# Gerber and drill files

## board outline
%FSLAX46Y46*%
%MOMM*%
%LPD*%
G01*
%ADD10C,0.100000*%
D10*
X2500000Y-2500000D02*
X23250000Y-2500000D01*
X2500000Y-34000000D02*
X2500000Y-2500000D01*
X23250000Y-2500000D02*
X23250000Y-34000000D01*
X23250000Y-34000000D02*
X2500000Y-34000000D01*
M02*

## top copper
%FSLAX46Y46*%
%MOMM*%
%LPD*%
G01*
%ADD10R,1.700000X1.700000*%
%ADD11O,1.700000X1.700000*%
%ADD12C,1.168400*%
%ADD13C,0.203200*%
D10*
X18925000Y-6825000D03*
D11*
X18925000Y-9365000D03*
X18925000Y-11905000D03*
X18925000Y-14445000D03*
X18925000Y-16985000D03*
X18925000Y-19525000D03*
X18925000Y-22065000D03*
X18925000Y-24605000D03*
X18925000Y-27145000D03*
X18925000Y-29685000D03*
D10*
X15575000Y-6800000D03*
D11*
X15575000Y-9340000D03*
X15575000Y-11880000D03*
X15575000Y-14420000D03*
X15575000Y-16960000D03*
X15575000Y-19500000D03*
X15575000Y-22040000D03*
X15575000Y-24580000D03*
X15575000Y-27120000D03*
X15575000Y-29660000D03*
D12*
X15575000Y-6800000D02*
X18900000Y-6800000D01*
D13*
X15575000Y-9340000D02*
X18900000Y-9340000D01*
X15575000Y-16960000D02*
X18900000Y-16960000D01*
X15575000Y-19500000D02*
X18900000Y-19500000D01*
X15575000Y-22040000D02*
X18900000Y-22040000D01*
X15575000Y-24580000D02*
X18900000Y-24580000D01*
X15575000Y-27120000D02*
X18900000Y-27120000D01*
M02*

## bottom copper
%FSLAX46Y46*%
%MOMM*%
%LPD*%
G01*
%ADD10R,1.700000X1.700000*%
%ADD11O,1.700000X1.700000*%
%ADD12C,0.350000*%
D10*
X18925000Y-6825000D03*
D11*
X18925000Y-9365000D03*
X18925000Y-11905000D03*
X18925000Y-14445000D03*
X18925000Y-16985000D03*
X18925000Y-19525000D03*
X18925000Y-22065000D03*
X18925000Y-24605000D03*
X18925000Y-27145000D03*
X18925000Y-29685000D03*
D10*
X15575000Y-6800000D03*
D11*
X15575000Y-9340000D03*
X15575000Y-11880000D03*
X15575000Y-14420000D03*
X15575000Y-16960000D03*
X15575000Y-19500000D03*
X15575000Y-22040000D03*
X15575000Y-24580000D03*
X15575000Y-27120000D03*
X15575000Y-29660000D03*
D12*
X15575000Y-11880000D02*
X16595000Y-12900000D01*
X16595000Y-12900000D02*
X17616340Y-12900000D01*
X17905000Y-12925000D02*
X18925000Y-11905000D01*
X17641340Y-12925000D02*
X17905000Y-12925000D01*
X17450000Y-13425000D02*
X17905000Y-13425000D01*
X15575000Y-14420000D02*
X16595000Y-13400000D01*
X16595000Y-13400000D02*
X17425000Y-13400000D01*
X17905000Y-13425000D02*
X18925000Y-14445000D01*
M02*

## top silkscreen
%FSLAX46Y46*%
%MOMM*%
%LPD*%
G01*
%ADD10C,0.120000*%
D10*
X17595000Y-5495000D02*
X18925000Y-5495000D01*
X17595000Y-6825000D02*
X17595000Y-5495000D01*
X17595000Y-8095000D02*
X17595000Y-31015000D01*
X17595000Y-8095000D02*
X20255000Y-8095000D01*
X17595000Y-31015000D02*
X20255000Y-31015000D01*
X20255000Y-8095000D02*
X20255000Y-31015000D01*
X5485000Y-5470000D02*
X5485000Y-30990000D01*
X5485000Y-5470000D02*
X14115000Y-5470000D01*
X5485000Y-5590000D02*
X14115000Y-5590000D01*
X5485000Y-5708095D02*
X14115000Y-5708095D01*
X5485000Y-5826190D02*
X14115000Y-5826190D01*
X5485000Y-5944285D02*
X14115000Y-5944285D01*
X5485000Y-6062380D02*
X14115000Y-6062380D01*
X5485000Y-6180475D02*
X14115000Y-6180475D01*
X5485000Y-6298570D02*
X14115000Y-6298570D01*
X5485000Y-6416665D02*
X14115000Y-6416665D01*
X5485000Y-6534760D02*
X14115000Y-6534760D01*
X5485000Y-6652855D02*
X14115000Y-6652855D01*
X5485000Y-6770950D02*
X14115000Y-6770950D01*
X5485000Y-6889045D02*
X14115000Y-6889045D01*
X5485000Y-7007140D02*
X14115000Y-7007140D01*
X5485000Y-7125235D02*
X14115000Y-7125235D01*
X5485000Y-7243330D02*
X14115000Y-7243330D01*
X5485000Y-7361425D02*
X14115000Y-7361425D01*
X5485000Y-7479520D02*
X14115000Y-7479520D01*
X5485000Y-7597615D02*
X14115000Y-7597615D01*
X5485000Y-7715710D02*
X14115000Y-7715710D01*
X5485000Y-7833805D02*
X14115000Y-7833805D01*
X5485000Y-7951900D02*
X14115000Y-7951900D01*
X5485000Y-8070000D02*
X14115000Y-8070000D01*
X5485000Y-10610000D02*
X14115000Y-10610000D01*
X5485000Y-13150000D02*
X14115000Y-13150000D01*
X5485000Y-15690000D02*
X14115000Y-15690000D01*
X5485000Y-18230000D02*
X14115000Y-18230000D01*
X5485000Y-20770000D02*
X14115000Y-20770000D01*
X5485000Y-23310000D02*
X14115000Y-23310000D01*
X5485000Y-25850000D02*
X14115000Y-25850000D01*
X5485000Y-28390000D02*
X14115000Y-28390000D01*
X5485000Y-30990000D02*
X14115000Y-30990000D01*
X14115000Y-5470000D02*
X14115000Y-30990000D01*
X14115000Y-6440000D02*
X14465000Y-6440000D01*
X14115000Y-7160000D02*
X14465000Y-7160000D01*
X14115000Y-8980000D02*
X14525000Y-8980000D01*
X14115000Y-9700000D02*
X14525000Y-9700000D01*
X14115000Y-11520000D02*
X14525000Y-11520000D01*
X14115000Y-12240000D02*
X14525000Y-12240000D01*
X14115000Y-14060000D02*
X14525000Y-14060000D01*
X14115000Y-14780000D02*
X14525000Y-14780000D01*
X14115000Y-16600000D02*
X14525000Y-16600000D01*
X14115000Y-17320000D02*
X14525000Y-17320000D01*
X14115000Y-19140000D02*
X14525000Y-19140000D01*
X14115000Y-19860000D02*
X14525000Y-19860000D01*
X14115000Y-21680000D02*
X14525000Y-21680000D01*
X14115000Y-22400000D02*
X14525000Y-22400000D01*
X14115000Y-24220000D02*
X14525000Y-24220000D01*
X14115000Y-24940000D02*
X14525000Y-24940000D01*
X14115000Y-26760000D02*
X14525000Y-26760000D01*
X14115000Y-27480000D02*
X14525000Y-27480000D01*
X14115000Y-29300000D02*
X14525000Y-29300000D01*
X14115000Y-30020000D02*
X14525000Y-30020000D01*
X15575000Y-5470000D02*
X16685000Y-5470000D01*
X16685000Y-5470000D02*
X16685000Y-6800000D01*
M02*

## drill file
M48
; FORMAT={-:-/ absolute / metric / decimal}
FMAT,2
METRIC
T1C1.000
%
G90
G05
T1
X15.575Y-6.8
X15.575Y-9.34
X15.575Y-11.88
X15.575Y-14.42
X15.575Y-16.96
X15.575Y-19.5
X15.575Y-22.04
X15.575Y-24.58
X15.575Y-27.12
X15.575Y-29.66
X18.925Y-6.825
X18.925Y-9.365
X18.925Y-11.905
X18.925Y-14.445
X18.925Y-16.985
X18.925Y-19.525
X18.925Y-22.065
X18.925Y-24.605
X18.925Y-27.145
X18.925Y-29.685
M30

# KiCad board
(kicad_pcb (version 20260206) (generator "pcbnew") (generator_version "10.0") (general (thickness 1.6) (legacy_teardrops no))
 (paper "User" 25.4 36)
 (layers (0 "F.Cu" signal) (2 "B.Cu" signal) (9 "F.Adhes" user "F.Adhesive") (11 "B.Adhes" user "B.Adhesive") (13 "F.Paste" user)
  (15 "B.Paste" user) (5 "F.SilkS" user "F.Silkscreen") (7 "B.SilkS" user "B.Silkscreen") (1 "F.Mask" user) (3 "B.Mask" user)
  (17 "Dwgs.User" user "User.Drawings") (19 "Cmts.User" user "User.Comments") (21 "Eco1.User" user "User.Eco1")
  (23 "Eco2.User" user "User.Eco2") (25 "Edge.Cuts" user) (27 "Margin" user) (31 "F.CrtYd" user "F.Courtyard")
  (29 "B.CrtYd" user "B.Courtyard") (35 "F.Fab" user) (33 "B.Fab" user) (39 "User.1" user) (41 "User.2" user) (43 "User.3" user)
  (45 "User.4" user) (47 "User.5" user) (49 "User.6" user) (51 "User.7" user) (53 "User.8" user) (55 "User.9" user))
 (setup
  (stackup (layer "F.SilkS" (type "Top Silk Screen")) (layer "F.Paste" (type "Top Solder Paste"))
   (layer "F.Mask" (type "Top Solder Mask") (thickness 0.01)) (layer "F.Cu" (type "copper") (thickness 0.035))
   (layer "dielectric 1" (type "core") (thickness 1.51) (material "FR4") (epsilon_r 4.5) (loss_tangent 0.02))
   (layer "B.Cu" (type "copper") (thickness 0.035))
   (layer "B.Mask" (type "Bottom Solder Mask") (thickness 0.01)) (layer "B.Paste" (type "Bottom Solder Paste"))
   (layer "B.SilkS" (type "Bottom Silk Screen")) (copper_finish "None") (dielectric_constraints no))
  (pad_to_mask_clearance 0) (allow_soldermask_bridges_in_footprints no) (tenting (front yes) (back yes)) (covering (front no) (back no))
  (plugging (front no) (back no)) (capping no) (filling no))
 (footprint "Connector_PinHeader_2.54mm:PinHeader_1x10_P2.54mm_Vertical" (layer "F.Cu") (at 18.925 6.825)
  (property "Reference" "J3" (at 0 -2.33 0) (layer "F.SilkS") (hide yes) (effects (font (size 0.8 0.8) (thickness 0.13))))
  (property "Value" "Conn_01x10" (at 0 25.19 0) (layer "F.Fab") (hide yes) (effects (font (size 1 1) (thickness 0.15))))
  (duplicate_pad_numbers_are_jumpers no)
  (fp_line (start -1.33 -1.33) (end 0 -1.33) (stroke (width 0.12) (type solid)) (layer "F.SilkS"))
  (fp_line (start -1.33 0) (end -1.33 -1.33) (stroke (width 0.12) (type solid)) (layer "F.SilkS"))
  (fp_line (start -1.33 1.27) (end -1.33 24.19) (stroke (width 0.12) (type solid)) (layer "F.SilkS"))
  (fp_line (start -1.33 1.27) (end 1.33 1.27) (stroke (width 0.12) (type solid)) (layer "F.SilkS"))
  (fp_line (start -1.33 24.19) (end 1.33 24.19) (stroke (width 0.12) (type solid)) (layer "F.SilkS"))
  (fp_line (start 1.33 1.27) (end 1.33 24.19) (stroke (width 0.12) (type solid)) (layer "F.SilkS"))
  (pad "1" thru_hole rect (at 0 0) (size 1.7 1.7) (drill 1) (layers "*.Cu" "*.Mask") (remove_unused_layers no) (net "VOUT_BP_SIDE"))
  (pad "2" thru_hole oval (at 0 2.54) (size 1.7 1.7) (drill 1) (layers "*.Cu" "*.Mask") (remove_unused_layers no) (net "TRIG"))
  (pad "3" thru_hole oval (at 0 5.08) (size 1.7 1.7) (drill 1) (layers "*.Cu" "*.Mask") (remove_unused_layers no) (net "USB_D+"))
  (pad "4" thru_hole oval (at 0 7.62) (size 1.7 1.7) (drill 1) (layers "*.Cu" "*.Mask") (remove_unused_layers no) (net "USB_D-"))
  (pad "5" thru_hole oval (at 0 10.16) (size 1.7 1.7) (drill 1) (layers "*.Cu" "*.Mask") (remove_unused_layers no) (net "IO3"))
  (pad "6" thru_hole oval (at 0 12.7) (size 1.7 1.7) (drill 1) (layers "*.Cu" "*.Mask") (remove_unused_layers no) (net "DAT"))
  (pad "7" thru_hole oval (at 0 15.24) (size 1.7 1.7) (drill 1) (layers "*.Cu" "*.Mask") (remove_unused_layers no) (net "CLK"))
  (pad "8" thru_hole oval (at 0 17.78) (size 1.7 1.7) (drill 1) (layers "*.Cu" "*.Mask") (remove_unused_layers no) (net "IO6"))
  (pad "9" thru_hole oval (at 0 20.32) (size 1.7 1.7) (drill 1) (layers "*.Cu" "*.Mask") (remove_unused_layers no) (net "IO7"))
  (pad "10" thru_hole oval (at 0 22.86) (size 1.7 1.7) (drill 1) (layers "*.Cu" "*.Mask") (remove_unused_layers no) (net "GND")))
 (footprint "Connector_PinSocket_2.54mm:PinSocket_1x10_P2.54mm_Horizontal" (layer "F.Cu") (at 15.575 6.8)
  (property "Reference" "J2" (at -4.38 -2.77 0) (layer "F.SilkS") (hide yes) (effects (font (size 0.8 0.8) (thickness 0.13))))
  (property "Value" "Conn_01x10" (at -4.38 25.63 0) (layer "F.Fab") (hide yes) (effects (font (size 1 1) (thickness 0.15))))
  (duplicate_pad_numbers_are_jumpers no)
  (fp_line (start -10.09 -1.33) (end -10.09 24.19) (stroke (width 0.12) (type solid)) (layer "F.SilkS"))
  (fp_line (start -10.09 -1.33) (end -1.46 -1.33) (stroke (width 0.12) (type solid)) (layer "F.SilkS"))
  (fp_line (start -10.09 -1.21) (end -1.46 -1.21) (stroke (width 0.12) (type solid)) (layer "F.SilkS"))
  (fp_line (start -10.09 -1.091905) (end -1.46 -1.091905) (stroke (width 0.12) (type solid)) (layer "F.SilkS"))
  (fp_line (start -10.09 -0.97381) (end -1.46 -0.97381) (stroke (width 0.12) (type solid)) (layer "F.SilkS"))
  (fp_line (start -10.09 -0.855715) (end -1.46 -0.855715) (stroke (width 0.12) (type solid)) (layer "F.SilkS"))
  (fp_line (start -10.09 -0.73762) (end -1.46 -0.73762) (stroke (width 0.12) (type solid)) (layer "F.SilkS"))
  (fp_line (start -10.09 -0.619525) (end -1.46 -0.619525) (stroke (width 0.12) (type solid)) (layer "F.SilkS"))
  (fp_line (start -10.09 -0.50143) (end -1.46 -0.50143) (stroke (width 0.12) (type solid)) (layer "F.SilkS"))
  (fp_line (start -10.09 -0.383335) (end -1.46 -0.383335) (stroke (width 0.12) (type solid)) (layer "F.SilkS"))
  (fp_line (start -10.09 -0.26524) (end -1.46 -0.26524) (stroke (width 0.12) (type solid)) (layer "F.SilkS"))
  (fp_line (start -10.09 -0.147145) (end -1.46 -0.147145) (stroke (width 0.12) (type solid)) (layer "F.SilkS"))
  (fp_line (start -10.09 -0.02905) (end -1.46 -0.02905) (stroke (width 0.12) (type solid)) (layer "F.SilkS"))
  (fp_line (start -10.09 0.089045) (end -1.46 0.089045) (stroke (width 0.12) (type solid)) (layer "F.SilkS"))
  (fp_line (start -10.09 0.20714) (end -1.46 0.20714) (stroke (width 0.12) (type solid)) (layer "F.SilkS"))
  (fp_line (start -10.09 0.325235) (end -1.46 0.325235) (stroke (width 0.12) (type solid)) (layer "F.SilkS"))
  (fp_line (start -10.09 0.44333) (end -1.46 0.44333) (stroke (width 0.12) (type solid)) (layer "F.SilkS"))
  (fp_line (start -10.09 0.561425) (end -1.46 0.561425) (stroke (width 0.12) (type solid)) (layer "F.SilkS"))
  (fp_line (start -10.09 0.67952) (end -1.46 0.67952) (stroke (width 0.12) (type solid)) (layer "F.SilkS"))
  (fp_line (start -10.09 0.797615) (end -1.46 0.797615) (stroke (width 0.12) (type solid)) (layer "F.SilkS"))
  (fp_line (start -10.09 0.91571) (end -1.46 0.91571) (stroke (width 0.12) (type solid)) (layer "F.SilkS"))
  (fp_line (start -10.09 1.033805) (end -1.46 1.033805) (stroke (width 0.12) (type solid)) (layer "F.SilkS"))
  (fp_line (start -10.09 1.1519) (end -1.46 1.1519) (stroke (width 0.12) (type solid)) (layer "F.SilkS"))
  (fp_line (start -10.09 1.27) (end -1.46 1.27) (stroke (width 0.12) (type solid)) (layer "F.SilkS"))
  (fp_line (start -10.09 3.81) (end -1.46 3.81) (stroke (width 0.12) (type solid)) (layer "F.SilkS"))
  (fp_line (start -10.09 6.35) (end -1.46 6.35) (stroke (width 0.12) (type solid)) (layer "F.SilkS"))
  (fp_line (start -10.09 8.89) (end -1.46 8.89) (stroke (width 0.12) (type solid)) (layer "F.SilkS"))
  (fp_line (start -10.09 11.43) (end -1.46 11.43) (stroke (width 0.12) (type solid)) (layer "F.SilkS"))
  (fp_line (start -10.09 13.97) (end -1.46 13.97) (stroke (width 0.12) (type solid)) (layer "F.SilkS"))
  (fp_line (start -10.09 16.51) (end -1.46 16.51) (stroke (width 0.12) (type solid)) (layer "F.SilkS"))
  (fp_line (start -10.09 19.05) (end -1.46 19.05) (stroke (width 0.12) (type solid)) (layer "F.SilkS"))
  (fp_line (start -10.09 21.59) (end -1.46 21.59) (stroke (width 0.12) (type solid)) (layer "F.SilkS"))
  (fp_line (start -10.09 24.19) (end -1.46 24.19) (stroke (width 0.12) (type solid)) (layer "F.SilkS"))
  (fp_line (start -1.46 -1.33) (end -1.46 24.19) (stroke (width 0.12) (type solid)) (layer "F.SilkS"))
  (fp_line (start -1.46 -0.36) (end -1.11 -0.36) (stroke (width 0.12) (type solid)) (layer "F.SilkS"))
  (fp_line (start -1.46 0.36) (end -1.11 0.36) (stroke (width 0.12) (type solid)) (layer "F.SilkS"))
  (fp_line (start -1.46 2.18) (end -1.05 2.18) (stroke (width 0.12) (type solid)) (layer "F.SilkS"))
  (fp_line (start -1.46 2.9) (end -1.05 2.9) (stroke (width 0.12) (type solid)) (layer "F.SilkS"))
  (fp_line (start -1.46 4.72) (end -1.05 4.72) (stroke (width 0.12) (type solid)) (layer "F.SilkS"))
  (fp_line (start -1.46 5.44) (end -1.05 5.44) (stroke (width 0.12) (type solid)) (layer "F.SilkS"))
  (fp_line (start -1.46 7.26) (end -1.05 7.26) (stroke (width 0.12) (type solid)) (layer "F.SilkS"))
  (fp_line (start -1.46 7.98) (end -1.05 7.98) (stroke (width 0.12) (type solid)) (layer "F.SilkS"))
  (fp_line (start -1.46 9.8) (end -1.05 9.8) (stroke (width 0.12) (type solid)) (layer "F.SilkS"))
  (fp_line (start -1.46 10.52) (end -1.05 10.52) (stroke (width 0.12) (type solid)) (layer "F.SilkS"))
  (fp_line (start -1.46 12.34) (end -1.05 12.34) (stroke (width 0.12) (type solid)) (layer "F.SilkS"))
  (fp_line (start -1.46 13.06) (end -1.05 13.06) (stroke (width 0.12) (type solid)) (layer "F.SilkS"))
  (fp_line (start -1.46 14.88) (end -1.05 14.88) (stroke (width 0.12) (type solid)) (layer "F.SilkS"))
  (fp_line (start -1.46 15.6) (end -1.05 15.6) (stroke (width 0.12) (type solid)) (layer "F.SilkS"))
  (fp_line (start -1.46 17.42) (end -1.05 17.42) (stroke (width 0.12) (type solid)) (layer "F.SilkS"))
  (fp_line (start -1.46 18.14) (end -1.05 18.14) (stroke (width 0.12) (type solid)) (layer "F.SilkS"))
  (fp_line (start -1.46 19.96) (end -1.05 19.96) (stroke (width 0.12) (type solid)) (layer "F.SilkS"))
  (fp_line (start -1.46 20.68) (end -1.05 20.68) (stroke (width 0.12) (type solid)) (layer "F.SilkS"))
  (fp_line (start -1.46 22.5) (end -1.05 22.5) (stroke (width 0.12) (type solid)) (layer "F.SilkS"))
  (fp_line (start -1.46 23.22) (end -1.05 23.22) (stroke (width 0.12) (type solid)) (layer "F.SilkS"))
  (fp_line (start 0 -1.33) (end 1.11 -1.33) (stroke (width 0.12) (type solid)) (layer "F.SilkS"))
  (fp_line (start 1.11 -1.33) (end 1.11 0) (stroke (width 0.12) (type solid)) (layer "F.SilkS"))
  (pad "1" thru_hole rect (at 0 0) (size 1.7 1.7) (drill 1) (layers "*.Cu" "*.Mask") (remove_unused_layers no) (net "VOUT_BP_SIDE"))
  (pad "2" thru_hole oval (at 0 2.54) (size 1.7 1.7) (drill 1) (layers "*.Cu" "*.Mask") (remove_unused_layers no) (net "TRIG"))
  (pad "3" thru_hole oval (at 0 5.08) (size 1.7 1.7) (drill 1) (layers "*.Cu" "*.Mask") (remove_unused_layers no) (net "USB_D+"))
  (pad "4" thru_hole oval (at 0 7.62) (size 1.7 1.7) (drill 1) (layers "*.Cu" "*.Mask") (remove_unused_layers no) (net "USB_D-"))
  (pad "5" thru_hole oval (at 0 10.16) (size 1.7 1.7) (drill 1) (layers "*.Cu" "*.Mask") (remove_unused_layers no) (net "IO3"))
  (pad "6" thru_hole oval (at 0 12.7) (size 1.7 1.7) (drill 1) (layers "*.Cu" "*.Mask") (remove_unused_layers no) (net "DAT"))
  (pad "7" thru_hole oval (at 0 15.24) (size 1.7 1.7) (drill 1) (layers "*.Cu" "*.Mask") (remove_unused_layers no) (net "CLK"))
  (pad "8" thru_hole oval (at 0 17.78) (size 1.7 1.7) (drill 1) (layers "*.Cu" "*.Mask") (remove_unused_layers no) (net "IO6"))
  (pad "9" thru_hole oval (at 0 20.32) (size 1.7 1.7) (drill 1) (layers "*.Cu" "*.Mask") (remove_unused_layers no) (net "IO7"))
  (pad "10" thru_hole oval (at 0 22.86) (size 1.7 1.7) (drill 1) (layers "*.Cu" "*.Mask") (remove_unused_layers no) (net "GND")))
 (gr_line (start 2.5 2.5) (end 23.25 2.5) (stroke (width 0.1) (type default)) (layer "Edge.Cuts"))
 (gr_line (start 2.5 34) (end 2.5 2.5) (stroke (width 0.1) (type default)) (layer "Edge.Cuts"))
 (gr_line (start 23.25 2.5) (end 23.25 34) (stroke (width 0.1) (type default)) (layer "Edge.Cuts"))
 (gr_line (start 23.25 34) (end 2.5 34) (stroke (width 0.1) (type default)) (layer "Edge.Cuts"))
 (segment (start 15.575 6.8) (end 18.9 6.8) (width 1.1684) (layer "F.Cu") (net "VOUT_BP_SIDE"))
 (segment (start 15.575 9.34) (end 18.9 9.34) (width 0.2032) (layer "F.Cu") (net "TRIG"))
 (segment (start 15.575 11.88) (end 16.595 12.9) (width 0.35) (layer "B.Cu") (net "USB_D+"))
 (segment (start 16.595 12.9) (end 17.61634 12.9) (width 0.35) (layer "B.Cu") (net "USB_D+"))
 (segment (start 17.905 12.925) (end 18.925 11.905) (width 0.35) (layer "B.Cu") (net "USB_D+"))
 (segment (start 17.64134 12.925) (end 17.905 12.925) (width 0.35) (layer "B.Cu") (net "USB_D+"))
 (segment (start 17.45 13.425) (end 17.905 13.425) (width 0.35) (layer "B.Cu") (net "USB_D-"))
 (segment (start 15.575 14.42) (end 16.595 13.4) (width 0.35) (layer "B.Cu") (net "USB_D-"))
 (segment (start 16.595 13.4) (end 17.425 13.4) (width 0.35) (layer "B.Cu") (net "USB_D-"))
 (segment (start 17.905 13.425) (end 18.925 14.445) (width 0.35) (layer "B.Cu") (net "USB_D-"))
 (segment (start 15.575 16.96) (end 18.9 16.96) (width 0.2032) (layer "F.Cu") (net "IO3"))
 (segment (start 15.575 19.5) (end 18.9 19.5) (width 0.2032) (layer "F.Cu") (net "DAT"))
 (segment (start 15.575 22.04) (end 18.9 22.04) (width 0.2032) (layer "F.Cu") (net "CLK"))
 (segment (start 15.575 24.58) (end 18.9 24.58) (width 0.2032) (layer "F.Cu") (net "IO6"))
 (segment (start 15.575 27.12) (end 18.9 27.12) (width 0.2032) (layer "F.Cu") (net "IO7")))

